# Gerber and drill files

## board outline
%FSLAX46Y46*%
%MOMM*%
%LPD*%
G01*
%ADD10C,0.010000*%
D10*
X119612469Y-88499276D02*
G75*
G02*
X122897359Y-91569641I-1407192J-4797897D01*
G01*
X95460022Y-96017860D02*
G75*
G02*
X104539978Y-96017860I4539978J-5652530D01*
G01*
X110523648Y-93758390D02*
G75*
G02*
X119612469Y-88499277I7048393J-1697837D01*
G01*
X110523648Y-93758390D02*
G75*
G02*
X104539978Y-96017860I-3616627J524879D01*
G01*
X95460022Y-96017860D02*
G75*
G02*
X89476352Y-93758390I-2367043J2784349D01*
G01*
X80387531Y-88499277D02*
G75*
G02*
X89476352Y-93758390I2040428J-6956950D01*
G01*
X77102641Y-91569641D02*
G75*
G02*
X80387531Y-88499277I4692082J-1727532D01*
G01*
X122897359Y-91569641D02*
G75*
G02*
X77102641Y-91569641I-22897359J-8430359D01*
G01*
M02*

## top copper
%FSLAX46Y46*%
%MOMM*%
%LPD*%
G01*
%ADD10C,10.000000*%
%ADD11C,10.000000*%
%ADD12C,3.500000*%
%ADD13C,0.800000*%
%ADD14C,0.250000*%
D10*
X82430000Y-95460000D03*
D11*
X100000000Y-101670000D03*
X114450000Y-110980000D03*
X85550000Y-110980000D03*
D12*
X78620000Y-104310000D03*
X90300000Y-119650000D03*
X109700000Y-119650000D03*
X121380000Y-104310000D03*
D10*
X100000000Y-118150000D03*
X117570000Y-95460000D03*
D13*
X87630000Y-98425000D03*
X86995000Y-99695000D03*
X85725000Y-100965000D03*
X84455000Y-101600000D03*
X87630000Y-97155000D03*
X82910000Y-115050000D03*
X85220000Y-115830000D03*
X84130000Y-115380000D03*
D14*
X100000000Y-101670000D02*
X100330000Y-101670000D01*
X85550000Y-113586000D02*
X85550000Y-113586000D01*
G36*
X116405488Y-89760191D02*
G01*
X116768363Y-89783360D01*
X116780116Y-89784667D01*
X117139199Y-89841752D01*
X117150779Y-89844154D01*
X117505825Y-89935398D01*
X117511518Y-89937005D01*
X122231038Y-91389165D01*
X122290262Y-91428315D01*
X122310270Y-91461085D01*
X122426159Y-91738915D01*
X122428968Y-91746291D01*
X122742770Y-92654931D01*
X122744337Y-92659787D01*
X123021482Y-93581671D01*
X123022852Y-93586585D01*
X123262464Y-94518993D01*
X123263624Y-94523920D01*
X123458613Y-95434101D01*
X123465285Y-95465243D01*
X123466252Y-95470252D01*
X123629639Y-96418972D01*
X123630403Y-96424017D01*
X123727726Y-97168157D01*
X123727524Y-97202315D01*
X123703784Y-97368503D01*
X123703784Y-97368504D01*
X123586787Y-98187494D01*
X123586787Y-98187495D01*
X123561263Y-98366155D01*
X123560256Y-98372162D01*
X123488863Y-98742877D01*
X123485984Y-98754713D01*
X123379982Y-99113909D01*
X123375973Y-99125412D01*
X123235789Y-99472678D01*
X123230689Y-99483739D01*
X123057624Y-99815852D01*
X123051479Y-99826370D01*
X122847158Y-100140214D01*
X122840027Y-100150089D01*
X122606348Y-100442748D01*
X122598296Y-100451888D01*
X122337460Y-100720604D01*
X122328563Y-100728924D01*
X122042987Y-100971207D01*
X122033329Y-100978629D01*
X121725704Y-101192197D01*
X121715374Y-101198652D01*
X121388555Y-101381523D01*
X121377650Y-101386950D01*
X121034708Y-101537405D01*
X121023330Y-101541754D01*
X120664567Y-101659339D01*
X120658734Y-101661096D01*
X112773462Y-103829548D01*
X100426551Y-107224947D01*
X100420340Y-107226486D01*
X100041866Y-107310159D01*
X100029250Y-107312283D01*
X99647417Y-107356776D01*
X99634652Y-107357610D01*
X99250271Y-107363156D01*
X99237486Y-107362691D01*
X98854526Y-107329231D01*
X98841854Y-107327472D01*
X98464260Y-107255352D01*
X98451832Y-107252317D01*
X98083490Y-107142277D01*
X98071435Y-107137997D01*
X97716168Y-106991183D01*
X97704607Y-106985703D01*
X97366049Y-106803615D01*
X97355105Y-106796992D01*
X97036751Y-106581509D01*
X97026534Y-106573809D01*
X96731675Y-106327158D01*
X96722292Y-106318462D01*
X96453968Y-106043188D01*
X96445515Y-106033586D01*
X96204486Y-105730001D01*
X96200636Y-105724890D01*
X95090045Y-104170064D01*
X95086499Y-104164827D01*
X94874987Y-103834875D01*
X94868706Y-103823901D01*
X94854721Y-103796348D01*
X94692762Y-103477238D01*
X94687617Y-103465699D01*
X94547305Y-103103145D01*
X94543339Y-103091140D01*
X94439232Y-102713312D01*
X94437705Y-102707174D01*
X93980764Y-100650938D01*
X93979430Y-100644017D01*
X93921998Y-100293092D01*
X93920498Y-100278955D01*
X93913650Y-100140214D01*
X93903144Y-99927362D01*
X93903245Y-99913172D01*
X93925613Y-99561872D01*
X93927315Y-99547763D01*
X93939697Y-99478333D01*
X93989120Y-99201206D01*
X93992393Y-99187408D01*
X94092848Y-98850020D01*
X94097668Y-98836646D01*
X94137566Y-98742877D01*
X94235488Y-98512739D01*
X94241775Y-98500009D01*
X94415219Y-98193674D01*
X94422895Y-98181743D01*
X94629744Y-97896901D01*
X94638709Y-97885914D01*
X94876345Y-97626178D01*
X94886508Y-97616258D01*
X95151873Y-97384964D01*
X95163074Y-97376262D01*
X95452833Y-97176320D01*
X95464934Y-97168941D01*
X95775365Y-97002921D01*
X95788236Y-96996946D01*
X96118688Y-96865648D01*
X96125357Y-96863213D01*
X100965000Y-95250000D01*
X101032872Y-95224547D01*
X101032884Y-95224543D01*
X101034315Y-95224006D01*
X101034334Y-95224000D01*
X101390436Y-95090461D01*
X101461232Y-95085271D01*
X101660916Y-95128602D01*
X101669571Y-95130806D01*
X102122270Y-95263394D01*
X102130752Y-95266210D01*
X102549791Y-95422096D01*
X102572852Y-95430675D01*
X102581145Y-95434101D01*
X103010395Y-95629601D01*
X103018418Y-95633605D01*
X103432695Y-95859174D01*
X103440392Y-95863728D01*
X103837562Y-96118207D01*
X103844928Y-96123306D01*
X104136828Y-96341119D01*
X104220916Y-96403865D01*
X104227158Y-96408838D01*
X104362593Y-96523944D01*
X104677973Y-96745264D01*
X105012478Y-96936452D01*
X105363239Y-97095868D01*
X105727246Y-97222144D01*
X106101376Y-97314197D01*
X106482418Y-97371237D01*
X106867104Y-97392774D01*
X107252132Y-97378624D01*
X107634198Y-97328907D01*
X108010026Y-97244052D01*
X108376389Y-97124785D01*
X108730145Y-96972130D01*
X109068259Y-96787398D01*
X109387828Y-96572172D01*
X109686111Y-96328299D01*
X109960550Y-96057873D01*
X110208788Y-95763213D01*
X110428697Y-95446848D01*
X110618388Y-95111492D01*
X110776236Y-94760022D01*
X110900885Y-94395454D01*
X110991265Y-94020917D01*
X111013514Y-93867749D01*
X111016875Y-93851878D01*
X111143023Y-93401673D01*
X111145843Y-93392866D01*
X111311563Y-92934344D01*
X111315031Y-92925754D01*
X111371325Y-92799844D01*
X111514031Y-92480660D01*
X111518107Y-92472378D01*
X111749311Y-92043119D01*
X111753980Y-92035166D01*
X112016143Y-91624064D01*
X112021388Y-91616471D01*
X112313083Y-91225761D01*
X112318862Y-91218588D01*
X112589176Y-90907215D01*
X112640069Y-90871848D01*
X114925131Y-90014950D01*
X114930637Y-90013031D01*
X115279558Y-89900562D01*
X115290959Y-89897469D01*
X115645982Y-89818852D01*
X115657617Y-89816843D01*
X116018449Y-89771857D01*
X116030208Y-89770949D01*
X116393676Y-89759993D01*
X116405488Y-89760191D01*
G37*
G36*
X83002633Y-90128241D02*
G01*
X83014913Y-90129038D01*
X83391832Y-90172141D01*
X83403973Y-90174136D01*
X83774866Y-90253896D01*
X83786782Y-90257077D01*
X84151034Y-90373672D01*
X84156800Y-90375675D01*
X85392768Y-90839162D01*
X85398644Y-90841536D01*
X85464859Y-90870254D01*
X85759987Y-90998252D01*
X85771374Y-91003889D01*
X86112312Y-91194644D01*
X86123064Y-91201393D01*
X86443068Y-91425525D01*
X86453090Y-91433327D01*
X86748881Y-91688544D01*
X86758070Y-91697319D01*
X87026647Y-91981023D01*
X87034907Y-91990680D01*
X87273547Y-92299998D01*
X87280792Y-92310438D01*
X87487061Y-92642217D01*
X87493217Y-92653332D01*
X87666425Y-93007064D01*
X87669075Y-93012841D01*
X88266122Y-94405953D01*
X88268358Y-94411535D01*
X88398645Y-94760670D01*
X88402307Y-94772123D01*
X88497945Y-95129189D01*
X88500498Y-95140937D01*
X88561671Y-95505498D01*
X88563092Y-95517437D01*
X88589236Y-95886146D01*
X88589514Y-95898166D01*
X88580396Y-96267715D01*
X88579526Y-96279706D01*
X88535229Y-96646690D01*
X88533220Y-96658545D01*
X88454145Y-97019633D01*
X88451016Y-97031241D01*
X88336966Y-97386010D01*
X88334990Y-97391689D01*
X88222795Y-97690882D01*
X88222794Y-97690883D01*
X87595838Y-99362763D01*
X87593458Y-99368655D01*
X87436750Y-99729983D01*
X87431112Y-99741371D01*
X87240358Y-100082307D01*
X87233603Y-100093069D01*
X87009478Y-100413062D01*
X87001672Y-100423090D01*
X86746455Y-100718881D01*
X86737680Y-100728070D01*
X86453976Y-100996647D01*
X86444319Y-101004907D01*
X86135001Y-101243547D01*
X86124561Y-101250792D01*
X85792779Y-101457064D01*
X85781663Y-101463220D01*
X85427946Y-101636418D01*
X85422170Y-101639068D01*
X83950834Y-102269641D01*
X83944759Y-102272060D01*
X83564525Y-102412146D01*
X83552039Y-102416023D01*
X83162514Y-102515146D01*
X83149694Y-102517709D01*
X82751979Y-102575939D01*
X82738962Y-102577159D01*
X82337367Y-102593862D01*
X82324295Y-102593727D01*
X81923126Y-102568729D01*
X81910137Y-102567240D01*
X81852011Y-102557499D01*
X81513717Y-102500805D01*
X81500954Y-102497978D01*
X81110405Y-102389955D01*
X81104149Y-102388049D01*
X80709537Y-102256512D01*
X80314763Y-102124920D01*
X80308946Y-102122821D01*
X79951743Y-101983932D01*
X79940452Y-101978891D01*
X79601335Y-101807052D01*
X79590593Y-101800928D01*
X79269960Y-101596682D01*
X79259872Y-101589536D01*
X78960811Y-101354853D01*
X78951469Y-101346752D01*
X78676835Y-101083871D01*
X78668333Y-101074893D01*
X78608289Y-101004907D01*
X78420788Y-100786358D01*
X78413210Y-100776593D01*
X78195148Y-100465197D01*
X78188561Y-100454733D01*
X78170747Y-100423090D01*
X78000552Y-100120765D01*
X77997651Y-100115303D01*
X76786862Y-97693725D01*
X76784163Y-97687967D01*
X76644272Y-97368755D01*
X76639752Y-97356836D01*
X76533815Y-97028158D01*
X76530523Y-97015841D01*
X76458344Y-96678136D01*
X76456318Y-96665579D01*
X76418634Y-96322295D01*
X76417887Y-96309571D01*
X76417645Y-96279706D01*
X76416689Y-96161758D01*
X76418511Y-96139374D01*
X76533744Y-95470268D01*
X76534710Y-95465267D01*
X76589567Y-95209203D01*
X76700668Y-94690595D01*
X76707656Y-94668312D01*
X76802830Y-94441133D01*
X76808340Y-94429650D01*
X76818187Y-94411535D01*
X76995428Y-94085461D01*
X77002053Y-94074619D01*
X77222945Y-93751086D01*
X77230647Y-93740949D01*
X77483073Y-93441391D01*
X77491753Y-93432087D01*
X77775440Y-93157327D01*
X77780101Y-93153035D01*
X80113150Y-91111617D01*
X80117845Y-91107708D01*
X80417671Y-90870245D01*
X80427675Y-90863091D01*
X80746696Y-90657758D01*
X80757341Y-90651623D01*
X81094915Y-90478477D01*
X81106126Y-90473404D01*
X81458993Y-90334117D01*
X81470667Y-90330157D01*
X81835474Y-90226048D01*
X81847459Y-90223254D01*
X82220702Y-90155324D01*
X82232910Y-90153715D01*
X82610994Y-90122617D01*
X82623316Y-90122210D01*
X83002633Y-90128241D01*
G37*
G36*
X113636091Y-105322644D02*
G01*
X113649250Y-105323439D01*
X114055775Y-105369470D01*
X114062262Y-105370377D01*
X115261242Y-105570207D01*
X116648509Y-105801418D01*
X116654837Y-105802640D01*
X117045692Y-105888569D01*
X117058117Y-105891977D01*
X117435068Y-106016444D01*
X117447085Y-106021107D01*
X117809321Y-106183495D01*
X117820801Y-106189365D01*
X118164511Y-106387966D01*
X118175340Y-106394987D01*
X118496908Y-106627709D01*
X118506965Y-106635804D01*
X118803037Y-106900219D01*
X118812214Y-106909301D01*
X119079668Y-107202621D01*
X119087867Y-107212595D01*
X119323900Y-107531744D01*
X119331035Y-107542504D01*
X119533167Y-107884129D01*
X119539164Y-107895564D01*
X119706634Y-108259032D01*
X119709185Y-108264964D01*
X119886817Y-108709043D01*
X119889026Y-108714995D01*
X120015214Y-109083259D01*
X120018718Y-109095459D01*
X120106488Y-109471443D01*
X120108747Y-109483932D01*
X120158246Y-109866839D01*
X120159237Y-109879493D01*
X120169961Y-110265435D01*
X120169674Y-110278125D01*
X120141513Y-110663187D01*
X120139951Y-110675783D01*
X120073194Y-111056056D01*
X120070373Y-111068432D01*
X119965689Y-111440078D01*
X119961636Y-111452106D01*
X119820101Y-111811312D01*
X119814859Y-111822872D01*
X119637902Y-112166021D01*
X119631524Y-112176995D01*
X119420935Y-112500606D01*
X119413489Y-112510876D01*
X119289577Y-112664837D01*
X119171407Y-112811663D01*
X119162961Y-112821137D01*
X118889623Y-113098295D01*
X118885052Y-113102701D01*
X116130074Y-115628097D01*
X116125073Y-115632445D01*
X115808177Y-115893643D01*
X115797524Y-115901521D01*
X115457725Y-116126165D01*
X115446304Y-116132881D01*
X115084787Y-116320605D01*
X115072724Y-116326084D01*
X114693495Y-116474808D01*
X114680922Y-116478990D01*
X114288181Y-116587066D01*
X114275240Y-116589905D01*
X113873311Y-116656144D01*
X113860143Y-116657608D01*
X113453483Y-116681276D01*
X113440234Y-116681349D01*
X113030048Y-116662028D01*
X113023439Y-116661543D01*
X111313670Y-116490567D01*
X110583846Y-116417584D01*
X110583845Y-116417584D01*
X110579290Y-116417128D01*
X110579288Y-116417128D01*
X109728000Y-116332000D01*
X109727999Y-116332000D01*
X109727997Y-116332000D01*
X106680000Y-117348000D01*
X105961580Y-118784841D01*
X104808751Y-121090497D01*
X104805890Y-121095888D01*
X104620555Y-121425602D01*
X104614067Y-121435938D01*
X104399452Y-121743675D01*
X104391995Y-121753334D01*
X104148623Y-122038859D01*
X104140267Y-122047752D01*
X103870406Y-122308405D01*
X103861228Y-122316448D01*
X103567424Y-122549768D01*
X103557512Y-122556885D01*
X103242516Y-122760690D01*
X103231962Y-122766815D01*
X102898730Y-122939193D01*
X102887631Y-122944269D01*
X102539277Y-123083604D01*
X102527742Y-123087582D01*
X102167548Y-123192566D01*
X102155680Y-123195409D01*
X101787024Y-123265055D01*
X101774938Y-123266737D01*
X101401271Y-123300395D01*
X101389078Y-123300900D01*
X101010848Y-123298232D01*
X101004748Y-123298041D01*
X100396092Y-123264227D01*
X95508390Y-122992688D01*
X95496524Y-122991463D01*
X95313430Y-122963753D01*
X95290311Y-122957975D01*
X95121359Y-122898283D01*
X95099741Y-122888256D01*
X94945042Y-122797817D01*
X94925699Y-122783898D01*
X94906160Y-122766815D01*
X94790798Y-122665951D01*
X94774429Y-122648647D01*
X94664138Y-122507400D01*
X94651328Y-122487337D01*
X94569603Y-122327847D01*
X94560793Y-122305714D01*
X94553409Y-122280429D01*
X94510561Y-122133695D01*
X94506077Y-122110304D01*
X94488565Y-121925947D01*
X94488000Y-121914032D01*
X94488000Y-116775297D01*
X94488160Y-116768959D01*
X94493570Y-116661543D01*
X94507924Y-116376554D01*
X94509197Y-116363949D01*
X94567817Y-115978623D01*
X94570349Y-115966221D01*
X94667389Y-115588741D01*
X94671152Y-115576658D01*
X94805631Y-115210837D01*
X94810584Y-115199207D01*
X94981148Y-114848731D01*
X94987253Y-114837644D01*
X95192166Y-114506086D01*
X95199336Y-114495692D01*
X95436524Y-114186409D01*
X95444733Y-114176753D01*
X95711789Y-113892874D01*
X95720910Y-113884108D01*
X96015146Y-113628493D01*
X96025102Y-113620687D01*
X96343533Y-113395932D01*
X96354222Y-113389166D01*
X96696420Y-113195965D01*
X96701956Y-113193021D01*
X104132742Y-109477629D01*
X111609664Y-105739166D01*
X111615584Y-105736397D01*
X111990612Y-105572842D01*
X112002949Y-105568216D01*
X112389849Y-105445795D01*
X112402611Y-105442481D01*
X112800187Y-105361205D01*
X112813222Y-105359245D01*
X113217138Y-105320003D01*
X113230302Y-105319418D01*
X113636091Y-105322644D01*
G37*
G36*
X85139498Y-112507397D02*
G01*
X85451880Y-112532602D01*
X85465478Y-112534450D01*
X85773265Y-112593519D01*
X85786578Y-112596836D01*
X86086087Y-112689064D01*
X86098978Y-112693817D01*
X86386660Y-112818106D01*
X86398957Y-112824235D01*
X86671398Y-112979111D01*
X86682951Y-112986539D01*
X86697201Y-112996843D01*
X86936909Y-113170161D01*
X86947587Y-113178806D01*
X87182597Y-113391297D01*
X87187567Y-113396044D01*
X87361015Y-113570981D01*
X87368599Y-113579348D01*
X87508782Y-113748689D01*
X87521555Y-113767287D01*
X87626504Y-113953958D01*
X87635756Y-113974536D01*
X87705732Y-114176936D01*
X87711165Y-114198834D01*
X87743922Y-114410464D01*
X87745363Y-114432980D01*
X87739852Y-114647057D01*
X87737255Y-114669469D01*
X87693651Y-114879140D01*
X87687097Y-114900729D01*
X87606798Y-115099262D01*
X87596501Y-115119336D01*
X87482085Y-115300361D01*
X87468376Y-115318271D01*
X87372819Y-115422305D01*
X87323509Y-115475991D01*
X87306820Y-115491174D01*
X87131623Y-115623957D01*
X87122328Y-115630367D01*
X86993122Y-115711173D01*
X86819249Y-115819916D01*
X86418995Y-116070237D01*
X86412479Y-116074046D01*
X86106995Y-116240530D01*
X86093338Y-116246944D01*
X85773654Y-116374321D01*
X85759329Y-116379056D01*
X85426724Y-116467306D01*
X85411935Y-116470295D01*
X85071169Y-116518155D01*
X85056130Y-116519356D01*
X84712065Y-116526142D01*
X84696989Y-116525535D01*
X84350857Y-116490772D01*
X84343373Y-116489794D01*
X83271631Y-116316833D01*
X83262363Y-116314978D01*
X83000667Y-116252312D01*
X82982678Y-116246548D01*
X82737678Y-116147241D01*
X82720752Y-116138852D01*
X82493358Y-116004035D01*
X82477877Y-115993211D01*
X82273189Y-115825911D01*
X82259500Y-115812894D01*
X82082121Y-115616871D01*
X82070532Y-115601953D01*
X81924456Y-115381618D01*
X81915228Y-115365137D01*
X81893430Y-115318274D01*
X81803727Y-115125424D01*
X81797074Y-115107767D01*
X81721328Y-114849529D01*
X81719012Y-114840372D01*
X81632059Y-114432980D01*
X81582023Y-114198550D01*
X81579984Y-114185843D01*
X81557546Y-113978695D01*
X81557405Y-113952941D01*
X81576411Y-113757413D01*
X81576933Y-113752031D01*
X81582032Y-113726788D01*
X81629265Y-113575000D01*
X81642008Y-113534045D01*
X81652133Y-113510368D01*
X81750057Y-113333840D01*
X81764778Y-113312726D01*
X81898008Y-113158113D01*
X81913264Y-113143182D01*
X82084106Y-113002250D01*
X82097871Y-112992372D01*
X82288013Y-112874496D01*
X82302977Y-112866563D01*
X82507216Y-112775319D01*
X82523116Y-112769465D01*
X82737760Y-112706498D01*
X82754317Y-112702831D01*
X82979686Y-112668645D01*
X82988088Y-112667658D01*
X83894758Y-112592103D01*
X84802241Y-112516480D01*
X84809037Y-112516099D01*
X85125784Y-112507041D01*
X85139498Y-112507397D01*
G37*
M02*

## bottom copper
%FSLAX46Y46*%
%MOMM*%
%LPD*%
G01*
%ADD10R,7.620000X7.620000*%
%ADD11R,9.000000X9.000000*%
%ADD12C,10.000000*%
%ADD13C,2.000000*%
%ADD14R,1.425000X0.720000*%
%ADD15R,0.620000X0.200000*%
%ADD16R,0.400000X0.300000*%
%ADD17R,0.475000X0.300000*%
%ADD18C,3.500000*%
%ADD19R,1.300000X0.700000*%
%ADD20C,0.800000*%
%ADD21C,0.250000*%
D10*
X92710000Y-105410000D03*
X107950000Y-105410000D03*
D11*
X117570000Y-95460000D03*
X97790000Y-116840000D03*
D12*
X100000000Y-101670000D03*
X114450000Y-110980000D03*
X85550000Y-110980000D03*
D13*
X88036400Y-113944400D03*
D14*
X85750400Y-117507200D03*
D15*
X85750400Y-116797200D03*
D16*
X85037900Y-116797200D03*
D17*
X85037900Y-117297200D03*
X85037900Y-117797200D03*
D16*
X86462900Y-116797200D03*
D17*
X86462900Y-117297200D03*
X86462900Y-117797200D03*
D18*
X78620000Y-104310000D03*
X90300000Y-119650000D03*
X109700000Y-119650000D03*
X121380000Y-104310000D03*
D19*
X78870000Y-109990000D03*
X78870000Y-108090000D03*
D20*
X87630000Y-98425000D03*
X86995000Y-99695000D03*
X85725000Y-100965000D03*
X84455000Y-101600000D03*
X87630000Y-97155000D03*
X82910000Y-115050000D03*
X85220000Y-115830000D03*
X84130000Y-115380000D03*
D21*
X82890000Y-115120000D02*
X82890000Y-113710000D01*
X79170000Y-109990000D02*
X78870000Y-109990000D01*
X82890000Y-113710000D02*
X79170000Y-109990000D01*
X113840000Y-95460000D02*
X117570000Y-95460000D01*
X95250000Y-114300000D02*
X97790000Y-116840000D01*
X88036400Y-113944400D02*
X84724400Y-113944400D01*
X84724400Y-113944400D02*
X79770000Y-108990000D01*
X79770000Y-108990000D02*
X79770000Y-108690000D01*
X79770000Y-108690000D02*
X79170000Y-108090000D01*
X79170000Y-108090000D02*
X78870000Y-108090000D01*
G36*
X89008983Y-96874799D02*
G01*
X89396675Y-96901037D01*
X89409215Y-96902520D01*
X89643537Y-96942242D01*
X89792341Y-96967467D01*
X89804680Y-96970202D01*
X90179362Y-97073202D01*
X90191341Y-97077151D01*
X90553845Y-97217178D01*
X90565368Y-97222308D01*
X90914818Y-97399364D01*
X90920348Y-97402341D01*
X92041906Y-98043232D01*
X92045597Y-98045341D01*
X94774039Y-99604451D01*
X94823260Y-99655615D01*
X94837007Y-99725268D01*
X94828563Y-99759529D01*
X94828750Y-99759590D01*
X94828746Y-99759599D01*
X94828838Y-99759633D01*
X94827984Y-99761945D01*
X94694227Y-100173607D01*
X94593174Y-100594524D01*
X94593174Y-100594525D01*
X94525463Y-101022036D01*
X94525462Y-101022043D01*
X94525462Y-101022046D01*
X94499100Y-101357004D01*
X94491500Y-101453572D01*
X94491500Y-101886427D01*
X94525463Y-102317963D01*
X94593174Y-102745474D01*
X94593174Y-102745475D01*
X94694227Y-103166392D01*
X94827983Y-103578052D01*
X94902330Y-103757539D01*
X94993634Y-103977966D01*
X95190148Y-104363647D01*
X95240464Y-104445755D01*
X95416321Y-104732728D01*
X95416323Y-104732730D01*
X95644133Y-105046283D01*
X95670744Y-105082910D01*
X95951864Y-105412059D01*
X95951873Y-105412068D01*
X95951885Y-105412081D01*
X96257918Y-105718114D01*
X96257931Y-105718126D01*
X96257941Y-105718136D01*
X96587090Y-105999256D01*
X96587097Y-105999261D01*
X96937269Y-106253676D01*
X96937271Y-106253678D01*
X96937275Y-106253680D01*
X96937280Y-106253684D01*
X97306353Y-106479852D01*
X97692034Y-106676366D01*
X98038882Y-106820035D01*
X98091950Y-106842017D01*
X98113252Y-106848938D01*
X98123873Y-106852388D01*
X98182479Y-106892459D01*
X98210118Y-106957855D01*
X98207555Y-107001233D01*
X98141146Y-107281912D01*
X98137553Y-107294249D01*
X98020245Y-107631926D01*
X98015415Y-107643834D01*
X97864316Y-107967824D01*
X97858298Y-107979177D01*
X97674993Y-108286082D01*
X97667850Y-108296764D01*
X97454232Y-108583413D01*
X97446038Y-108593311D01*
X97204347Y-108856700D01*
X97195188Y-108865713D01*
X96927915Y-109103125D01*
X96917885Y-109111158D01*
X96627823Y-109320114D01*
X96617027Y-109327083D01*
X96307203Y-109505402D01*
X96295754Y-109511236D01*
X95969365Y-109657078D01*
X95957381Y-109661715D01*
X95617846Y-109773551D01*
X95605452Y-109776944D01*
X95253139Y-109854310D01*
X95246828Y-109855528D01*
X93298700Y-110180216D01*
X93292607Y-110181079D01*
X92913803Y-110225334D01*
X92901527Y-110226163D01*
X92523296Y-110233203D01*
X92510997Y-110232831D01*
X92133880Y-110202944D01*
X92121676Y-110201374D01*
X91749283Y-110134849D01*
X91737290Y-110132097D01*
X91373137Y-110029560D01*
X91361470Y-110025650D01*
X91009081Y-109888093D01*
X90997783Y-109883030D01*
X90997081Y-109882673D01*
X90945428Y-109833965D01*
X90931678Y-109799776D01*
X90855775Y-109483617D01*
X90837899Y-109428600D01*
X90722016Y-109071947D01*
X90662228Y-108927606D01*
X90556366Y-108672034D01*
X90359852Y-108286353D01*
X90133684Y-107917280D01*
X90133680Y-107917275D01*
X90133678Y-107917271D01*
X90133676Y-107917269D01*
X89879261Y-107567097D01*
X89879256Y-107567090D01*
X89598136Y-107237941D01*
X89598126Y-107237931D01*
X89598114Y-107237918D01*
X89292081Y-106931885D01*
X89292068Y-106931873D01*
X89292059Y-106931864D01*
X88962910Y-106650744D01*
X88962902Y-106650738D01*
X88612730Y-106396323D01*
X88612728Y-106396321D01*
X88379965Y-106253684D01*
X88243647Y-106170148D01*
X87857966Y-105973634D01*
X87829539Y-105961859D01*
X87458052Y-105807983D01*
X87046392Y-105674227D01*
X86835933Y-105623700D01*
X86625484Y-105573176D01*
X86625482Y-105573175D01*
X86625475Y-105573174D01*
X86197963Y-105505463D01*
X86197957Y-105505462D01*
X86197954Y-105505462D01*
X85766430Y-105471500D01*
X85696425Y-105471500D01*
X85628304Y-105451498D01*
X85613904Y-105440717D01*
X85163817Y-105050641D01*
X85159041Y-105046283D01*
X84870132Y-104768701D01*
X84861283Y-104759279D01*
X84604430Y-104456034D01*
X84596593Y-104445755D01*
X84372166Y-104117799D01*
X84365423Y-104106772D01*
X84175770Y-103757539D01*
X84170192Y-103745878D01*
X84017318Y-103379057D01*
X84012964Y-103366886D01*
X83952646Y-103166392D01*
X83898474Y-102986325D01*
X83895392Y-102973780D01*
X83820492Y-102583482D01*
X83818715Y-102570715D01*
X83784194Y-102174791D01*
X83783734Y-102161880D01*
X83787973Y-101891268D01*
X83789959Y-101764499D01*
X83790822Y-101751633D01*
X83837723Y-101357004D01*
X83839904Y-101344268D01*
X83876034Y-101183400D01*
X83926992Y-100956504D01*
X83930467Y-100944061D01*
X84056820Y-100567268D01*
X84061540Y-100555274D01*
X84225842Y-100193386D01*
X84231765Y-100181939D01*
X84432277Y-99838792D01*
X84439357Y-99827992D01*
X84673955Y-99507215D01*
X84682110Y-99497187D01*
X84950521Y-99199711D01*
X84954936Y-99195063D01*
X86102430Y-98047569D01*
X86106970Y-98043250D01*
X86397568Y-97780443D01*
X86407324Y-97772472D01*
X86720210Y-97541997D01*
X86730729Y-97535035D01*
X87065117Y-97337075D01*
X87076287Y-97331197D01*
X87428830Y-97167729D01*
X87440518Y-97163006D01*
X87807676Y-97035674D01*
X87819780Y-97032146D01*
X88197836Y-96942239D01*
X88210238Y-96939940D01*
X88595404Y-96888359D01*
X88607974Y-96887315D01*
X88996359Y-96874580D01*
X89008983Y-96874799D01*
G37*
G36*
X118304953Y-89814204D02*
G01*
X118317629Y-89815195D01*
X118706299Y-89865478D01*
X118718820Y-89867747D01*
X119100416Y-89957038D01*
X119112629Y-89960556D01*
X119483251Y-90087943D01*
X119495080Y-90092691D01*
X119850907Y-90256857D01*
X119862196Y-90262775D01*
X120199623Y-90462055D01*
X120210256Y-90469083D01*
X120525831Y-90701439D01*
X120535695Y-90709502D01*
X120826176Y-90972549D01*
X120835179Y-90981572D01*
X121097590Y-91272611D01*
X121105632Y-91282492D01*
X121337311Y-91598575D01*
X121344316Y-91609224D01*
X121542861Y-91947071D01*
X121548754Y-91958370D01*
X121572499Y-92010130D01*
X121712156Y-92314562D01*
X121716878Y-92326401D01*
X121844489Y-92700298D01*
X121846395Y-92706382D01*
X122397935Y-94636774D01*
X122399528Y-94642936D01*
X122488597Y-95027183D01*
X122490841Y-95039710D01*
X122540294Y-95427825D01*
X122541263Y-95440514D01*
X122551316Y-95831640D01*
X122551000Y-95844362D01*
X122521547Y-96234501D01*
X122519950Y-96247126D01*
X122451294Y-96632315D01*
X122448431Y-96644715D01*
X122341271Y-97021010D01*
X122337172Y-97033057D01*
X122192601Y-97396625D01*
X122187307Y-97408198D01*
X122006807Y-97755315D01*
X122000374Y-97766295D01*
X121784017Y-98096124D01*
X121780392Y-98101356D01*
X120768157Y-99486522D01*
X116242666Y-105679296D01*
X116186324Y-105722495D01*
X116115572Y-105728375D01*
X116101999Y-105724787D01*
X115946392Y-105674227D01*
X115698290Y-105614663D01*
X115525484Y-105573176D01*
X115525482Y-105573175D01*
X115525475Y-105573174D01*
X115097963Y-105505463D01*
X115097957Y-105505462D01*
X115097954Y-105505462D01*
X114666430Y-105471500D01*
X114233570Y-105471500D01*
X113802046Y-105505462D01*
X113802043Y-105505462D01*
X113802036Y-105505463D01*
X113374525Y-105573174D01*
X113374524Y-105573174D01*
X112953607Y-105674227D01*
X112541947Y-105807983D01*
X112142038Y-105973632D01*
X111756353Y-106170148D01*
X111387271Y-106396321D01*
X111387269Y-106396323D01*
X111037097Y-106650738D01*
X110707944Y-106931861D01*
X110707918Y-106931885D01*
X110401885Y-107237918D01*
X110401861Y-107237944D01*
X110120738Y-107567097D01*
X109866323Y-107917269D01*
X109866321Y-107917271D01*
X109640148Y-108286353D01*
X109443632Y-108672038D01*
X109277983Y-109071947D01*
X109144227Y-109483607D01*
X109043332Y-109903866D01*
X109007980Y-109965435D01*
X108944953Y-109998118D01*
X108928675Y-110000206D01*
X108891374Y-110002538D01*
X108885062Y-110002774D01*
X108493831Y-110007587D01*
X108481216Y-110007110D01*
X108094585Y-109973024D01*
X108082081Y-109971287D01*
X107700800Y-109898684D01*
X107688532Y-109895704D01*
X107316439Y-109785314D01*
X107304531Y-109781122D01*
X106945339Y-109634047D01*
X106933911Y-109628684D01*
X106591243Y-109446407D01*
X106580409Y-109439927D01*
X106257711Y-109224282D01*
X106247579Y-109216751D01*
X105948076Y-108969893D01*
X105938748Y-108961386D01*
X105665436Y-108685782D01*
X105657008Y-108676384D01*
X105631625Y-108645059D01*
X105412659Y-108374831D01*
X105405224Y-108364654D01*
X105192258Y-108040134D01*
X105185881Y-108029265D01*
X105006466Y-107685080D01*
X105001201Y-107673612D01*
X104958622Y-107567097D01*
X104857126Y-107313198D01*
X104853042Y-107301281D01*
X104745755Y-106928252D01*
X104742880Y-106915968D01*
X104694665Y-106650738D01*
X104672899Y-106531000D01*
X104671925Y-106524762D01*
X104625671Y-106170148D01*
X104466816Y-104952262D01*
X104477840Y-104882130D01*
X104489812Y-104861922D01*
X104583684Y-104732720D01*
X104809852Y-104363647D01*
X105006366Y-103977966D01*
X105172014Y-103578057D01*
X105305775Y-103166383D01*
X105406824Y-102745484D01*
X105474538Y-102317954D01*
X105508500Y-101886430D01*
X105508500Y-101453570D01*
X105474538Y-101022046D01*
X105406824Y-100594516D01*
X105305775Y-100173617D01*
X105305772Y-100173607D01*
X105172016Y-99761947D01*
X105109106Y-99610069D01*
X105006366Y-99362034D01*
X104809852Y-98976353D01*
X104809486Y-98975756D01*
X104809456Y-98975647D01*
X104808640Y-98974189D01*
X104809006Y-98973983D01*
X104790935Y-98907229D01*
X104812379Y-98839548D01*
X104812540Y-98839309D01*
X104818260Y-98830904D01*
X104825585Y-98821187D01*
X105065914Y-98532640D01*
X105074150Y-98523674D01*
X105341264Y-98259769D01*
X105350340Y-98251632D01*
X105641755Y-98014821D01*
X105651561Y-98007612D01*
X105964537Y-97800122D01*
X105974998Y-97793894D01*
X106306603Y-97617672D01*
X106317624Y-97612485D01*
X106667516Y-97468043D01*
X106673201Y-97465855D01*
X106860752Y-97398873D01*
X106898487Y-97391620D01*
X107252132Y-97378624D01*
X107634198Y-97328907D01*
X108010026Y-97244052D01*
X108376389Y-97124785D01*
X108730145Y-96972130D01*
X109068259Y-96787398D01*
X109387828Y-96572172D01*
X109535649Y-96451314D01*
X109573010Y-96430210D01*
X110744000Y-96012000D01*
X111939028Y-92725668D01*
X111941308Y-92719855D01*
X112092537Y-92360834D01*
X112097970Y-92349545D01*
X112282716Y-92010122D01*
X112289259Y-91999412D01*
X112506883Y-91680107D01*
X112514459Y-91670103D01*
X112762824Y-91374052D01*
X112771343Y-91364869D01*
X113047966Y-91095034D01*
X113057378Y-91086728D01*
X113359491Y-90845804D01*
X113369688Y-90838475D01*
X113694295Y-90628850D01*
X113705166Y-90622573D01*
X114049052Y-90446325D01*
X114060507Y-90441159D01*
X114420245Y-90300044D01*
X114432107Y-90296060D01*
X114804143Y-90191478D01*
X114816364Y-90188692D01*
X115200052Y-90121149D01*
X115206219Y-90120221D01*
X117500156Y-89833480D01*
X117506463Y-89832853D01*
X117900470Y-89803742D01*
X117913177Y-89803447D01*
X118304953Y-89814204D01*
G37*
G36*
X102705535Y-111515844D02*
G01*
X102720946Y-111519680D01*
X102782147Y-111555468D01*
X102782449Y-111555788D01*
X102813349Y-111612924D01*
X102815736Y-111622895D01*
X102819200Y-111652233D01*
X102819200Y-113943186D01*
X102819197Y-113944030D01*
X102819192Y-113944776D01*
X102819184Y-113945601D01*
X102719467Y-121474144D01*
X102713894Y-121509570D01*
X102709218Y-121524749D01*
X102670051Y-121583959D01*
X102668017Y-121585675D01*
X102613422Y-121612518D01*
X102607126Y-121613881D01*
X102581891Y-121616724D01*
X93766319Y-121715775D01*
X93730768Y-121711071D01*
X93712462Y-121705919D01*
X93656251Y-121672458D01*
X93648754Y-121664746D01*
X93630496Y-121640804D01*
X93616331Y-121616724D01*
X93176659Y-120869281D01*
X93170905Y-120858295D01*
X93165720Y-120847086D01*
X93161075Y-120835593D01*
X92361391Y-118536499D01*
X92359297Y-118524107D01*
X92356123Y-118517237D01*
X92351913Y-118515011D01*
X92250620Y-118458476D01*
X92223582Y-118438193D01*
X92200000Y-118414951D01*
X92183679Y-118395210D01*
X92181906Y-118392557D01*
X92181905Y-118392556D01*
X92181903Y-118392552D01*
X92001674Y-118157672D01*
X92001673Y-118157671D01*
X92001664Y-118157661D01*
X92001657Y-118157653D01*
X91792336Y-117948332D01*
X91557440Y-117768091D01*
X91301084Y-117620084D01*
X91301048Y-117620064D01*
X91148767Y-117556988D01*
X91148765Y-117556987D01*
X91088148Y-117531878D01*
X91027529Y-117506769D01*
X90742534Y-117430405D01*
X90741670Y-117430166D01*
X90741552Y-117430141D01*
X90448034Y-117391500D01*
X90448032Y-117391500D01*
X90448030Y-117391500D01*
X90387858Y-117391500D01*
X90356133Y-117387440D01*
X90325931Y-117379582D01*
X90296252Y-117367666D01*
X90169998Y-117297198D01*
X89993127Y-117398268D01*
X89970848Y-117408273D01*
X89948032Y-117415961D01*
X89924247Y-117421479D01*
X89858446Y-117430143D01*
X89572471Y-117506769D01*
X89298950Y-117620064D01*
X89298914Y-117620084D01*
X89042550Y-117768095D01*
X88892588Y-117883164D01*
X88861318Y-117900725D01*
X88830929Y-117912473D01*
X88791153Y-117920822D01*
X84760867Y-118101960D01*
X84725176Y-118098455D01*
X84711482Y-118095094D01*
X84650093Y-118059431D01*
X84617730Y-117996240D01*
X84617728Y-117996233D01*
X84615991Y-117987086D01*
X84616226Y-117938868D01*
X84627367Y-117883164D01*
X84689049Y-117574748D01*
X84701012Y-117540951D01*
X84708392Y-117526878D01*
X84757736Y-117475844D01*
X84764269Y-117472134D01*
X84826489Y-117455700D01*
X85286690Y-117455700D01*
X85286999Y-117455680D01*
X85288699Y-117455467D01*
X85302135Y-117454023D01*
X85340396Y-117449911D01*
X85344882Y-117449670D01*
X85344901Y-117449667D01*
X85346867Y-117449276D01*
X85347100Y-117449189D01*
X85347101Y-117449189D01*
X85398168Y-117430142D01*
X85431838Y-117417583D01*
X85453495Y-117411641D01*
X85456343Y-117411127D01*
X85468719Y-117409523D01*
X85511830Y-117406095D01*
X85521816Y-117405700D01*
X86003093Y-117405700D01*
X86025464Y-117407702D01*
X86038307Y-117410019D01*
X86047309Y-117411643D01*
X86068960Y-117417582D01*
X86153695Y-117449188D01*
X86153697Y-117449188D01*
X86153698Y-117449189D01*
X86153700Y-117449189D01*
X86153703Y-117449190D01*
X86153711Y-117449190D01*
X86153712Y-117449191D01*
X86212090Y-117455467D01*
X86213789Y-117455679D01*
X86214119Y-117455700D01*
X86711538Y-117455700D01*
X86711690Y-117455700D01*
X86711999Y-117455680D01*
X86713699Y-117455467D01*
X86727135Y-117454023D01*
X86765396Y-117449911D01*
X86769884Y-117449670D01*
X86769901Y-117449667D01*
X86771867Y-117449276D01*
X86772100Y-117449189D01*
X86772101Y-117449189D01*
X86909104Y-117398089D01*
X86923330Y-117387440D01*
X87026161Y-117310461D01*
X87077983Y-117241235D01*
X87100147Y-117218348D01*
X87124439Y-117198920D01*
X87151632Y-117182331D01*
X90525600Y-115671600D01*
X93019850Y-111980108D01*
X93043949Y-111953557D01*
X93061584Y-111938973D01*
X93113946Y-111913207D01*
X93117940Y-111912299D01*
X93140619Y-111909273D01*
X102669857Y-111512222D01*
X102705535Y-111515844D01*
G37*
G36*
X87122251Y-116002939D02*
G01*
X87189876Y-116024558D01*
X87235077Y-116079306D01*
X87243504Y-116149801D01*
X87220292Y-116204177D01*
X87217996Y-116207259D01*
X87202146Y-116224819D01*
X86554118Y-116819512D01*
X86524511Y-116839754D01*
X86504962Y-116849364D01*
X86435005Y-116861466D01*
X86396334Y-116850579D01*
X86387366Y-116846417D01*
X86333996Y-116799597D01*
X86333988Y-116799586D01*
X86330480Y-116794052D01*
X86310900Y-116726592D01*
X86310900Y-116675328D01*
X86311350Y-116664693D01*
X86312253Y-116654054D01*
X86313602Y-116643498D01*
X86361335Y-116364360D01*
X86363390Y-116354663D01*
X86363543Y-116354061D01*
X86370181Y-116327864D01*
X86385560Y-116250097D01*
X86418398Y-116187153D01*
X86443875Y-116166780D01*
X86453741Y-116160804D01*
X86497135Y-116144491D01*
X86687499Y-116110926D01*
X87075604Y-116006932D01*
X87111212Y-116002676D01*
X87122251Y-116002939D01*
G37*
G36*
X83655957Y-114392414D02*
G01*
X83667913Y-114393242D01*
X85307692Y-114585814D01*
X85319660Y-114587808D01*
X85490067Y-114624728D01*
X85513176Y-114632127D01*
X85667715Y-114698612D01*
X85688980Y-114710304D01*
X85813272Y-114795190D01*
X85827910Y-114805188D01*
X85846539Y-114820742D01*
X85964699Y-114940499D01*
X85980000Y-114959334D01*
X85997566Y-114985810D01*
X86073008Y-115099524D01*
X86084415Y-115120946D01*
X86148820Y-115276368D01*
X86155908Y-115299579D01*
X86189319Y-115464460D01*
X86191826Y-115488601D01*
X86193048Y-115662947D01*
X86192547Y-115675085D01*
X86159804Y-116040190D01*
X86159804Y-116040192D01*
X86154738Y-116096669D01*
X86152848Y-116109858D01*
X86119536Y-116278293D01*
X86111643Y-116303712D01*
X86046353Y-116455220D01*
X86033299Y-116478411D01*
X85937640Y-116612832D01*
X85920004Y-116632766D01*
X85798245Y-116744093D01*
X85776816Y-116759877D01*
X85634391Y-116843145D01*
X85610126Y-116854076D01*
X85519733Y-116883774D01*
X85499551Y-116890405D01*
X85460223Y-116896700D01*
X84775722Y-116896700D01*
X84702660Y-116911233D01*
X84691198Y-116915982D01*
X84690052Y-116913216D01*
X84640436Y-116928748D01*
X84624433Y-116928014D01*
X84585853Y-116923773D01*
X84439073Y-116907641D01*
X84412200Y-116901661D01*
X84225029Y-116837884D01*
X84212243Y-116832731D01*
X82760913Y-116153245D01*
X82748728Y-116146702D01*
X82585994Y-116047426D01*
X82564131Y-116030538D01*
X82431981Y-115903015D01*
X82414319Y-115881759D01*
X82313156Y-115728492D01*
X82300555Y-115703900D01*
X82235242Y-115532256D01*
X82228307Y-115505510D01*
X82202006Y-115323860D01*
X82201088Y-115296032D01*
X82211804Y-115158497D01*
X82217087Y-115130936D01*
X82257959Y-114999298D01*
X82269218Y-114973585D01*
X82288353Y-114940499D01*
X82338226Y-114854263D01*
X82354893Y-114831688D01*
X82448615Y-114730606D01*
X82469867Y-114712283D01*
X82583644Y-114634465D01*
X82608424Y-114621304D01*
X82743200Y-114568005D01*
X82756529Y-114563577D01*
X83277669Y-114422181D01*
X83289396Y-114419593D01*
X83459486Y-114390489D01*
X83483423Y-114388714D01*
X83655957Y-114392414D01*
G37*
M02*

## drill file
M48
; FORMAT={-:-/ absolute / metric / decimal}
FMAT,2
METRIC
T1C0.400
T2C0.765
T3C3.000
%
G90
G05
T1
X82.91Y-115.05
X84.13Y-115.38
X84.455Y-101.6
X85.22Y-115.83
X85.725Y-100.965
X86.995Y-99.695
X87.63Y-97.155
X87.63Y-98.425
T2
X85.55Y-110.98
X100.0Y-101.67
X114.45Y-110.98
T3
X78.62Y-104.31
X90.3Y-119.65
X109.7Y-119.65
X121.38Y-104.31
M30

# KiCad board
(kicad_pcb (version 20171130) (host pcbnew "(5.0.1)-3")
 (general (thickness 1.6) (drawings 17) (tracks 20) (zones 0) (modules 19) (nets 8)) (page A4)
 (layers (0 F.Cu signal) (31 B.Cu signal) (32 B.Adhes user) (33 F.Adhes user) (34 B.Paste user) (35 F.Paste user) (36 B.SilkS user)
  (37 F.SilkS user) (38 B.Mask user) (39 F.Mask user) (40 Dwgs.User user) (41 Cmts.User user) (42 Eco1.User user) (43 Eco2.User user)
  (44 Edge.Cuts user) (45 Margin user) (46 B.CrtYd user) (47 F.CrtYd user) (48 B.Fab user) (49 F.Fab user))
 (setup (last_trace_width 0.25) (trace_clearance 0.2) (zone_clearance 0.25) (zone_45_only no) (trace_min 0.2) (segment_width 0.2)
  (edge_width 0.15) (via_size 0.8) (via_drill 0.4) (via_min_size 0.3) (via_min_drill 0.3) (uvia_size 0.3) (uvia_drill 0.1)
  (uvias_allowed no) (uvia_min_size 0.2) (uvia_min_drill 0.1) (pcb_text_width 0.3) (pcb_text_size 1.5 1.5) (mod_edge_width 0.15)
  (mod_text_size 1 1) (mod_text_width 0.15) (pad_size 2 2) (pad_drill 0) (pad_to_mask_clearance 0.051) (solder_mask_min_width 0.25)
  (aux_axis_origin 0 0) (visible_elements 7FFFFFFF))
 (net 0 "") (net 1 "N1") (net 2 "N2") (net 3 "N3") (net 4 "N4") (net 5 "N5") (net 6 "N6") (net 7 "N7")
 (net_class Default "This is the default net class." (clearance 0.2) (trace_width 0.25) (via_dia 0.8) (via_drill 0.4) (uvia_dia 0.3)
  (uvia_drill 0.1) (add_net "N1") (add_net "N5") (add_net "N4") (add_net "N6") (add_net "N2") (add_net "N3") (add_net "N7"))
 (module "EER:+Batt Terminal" (layer F.Cu) (at 82.43 95.46)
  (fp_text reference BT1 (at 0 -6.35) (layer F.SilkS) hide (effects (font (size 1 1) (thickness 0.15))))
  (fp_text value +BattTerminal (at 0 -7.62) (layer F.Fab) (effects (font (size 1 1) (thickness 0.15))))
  (pad 1 smd circle (at 0 0) (size 10 10) (layers F.Cu F.Paste F.Mask) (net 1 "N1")))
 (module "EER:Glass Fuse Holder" (layer F.Cu) (at 111.76 101.6 180)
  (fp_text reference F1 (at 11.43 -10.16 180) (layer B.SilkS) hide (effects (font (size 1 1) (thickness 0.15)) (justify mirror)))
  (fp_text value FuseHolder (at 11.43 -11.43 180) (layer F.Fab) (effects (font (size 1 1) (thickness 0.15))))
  (pad 2 smd rect (at 19.05 -3.81 180) (size 7.62 7.62) (layers B.Cu B.Mask) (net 1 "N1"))
  (pad 1 smd rect (at 3.81 -3.81 180) (size 7.62 7.62) (layers B.Cu B.Mask) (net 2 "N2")))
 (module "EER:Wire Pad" (layer F.Cu) (at 112.49 100.54)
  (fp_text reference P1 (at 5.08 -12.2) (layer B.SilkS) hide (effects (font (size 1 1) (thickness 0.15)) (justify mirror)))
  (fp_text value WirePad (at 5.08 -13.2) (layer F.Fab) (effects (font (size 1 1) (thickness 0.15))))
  (pad 1 smd rect (at 5.08 -5.08) (size 9 9) (layers B.Cu B.Mask) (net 2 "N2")))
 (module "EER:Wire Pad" (layer F.Cu) (at 92.71 121.92)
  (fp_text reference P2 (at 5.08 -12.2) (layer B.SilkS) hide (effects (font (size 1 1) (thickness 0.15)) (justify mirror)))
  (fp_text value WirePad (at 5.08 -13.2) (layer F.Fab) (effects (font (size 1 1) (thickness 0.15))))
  (pad 1 smd rect (at 5.08 -5.08) (size 9 9) (layers B.Cu B.Mask) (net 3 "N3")))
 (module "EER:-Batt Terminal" (layer F.Cu) (at 100 101.67)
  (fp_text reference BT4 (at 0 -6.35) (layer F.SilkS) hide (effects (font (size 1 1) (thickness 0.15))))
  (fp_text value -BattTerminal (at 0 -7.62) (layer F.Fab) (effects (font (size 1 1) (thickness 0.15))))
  (pad 1 thru_hole circle (at 0 0) (size 10 10) (drill 0.765) (layers F.Cu F.Mask) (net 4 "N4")))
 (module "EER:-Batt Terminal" (layer F.Cu) (at 114.45 110.98)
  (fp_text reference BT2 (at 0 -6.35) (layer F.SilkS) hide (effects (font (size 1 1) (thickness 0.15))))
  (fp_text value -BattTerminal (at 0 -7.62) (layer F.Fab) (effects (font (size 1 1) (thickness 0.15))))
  (pad 1 thru_hole circle (at 0 0) (size 10 10) (drill 0.765) (layers F.Cu F.Mask) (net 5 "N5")))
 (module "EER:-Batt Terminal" (layer F.Cu) (at 85.55 110.98)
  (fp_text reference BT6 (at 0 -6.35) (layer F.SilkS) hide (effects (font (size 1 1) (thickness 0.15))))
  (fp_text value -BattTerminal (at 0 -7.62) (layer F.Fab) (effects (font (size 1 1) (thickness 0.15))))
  (pad 1 thru_hole circle (at 0 0) (size 10 10) (drill 0.765) (layers F.Cu F.Mask) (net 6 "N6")))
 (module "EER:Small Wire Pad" (layer F.Cu) (at 85.4964 116.4844)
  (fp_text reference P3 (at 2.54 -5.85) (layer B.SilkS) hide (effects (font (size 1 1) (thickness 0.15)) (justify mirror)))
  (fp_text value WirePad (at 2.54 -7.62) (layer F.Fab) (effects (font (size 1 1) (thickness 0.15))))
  (pad 1 smd circle (at 2.54 -2.54) (size 2 2) (layers B.Cu B.Paste B.Mask) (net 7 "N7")))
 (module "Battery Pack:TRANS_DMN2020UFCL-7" (layer F.Cu) (at 85.7504 117.2972 180)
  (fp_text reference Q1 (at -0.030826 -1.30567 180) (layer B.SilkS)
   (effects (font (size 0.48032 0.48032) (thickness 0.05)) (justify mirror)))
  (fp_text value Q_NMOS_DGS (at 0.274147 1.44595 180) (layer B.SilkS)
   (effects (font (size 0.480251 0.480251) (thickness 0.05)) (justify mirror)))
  (pad 1 smd rect (at 0 -0.21 180) (size 1.425 0.72) (layers B.Cu B.Paste B.Mask) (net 3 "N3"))
  (pad 3 smd rect (at 0 0.5 180) (size 0.62 0.2) (layers B.Cu B.Paste B.Mask) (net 6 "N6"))
  (pad 3 smd rect (at 0.7125 0.5 180) (size 0.4 0.3) (layers B.Cu B.Paste B.Mask) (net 6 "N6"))
  (pad 1 smd rect (at 0.7125 0 180) (size 0.475 0.3) (layers B.Cu B.Paste B.Mask) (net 3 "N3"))
  (pad 1 smd rect (at 0.7125 -0.5 180) (size 0.475 0.3) (layers B.Cu B.Paste B.Mask) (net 3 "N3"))
  (pad 2 smd rect (at -0.7125 0.5 180) (size 0.4 0.3) (layers B.Cu B.Paste B.Mask) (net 7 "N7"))
  (pad 1 smd rect (at -0.7125 0 180) (size 0.475 0.3) (layers B.Cu B.Paste B.Mask) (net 3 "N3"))
  (pad 1 smd rect (at -0.7125 -0.5 180) (size 0.475 0.3) (layers B.Cu B.Paste B.Mask) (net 3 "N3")))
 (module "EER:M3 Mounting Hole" (layer F.Cu) (at 78.62 104.31)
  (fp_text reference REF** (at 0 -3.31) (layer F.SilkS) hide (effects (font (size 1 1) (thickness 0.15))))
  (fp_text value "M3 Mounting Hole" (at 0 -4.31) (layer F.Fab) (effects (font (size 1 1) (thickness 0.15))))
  (pad 1 thru_hole circle (at 0 0) (size 3.5 3.5) (drill 3) (layers *.Cu *.Mask)))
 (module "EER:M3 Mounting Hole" (layer F.Cu) (at 90.3 119.65)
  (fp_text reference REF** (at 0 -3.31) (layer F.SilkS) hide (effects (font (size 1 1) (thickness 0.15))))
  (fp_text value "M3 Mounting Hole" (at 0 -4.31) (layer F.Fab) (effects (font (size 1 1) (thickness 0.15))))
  (pad 1 thru_hole circle (at 0 0) (size 3.5 3.5) (drill 3) (layers *.Cu *.Mask)))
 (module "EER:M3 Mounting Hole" (layer F.Cu) (at 109.7 119.65)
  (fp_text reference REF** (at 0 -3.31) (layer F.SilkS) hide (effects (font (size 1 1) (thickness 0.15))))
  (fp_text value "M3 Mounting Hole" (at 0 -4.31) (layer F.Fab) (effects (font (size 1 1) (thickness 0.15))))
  (pad 1 thru_hole circle (at 0 0) (size 3.5 3.5) (drill 3) (layers *.Cu *.Mask)))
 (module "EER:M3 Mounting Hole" (layer F.Cu) (at 121.38 104.31)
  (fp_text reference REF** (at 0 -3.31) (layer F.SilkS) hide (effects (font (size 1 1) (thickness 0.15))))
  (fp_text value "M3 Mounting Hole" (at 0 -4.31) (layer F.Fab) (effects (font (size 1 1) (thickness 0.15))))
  (pad 1 thru_hole circle (at 0 0) (size 3.5 3.5) (drill 3) (layers *.Cu *.Mask)))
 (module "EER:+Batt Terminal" (layer F.Cu) (at 100 118.15)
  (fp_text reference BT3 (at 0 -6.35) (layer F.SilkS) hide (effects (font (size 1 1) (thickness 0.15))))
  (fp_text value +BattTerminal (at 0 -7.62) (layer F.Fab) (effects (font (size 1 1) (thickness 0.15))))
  (pad 1 smd circle (at 0 0) (size 10 10) (layers F.Cu F.Paste F.Mask) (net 5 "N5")))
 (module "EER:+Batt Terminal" (layer F.Cu) (at 117.57 95.46)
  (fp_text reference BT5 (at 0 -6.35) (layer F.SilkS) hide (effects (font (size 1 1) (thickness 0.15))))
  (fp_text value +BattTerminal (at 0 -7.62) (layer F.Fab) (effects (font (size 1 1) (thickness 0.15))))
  (pad 1 smd circle (at 0 0) (size 10 10) (layers F.Cu F.Paste F.Mask) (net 4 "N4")))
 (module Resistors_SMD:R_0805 (layer B.Cu) (at 78.87 109.04 270)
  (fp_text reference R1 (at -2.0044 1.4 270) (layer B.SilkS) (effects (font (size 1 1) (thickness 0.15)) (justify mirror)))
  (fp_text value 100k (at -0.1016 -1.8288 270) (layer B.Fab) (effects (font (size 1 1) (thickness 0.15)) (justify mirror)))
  (pad 2 smd rect (at 0.95 0 270) (size 0.7 1.3) (layers B.Cu B.Paste B.Mask) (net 6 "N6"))
  (pad 1 smd rect (at -0.95 0 270) (size 0.7 1.3) (layers B.Cu B.Paste B.Mask) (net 7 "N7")))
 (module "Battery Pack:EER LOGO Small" (layer B.Cu) (at 81.9912 91.2876 180)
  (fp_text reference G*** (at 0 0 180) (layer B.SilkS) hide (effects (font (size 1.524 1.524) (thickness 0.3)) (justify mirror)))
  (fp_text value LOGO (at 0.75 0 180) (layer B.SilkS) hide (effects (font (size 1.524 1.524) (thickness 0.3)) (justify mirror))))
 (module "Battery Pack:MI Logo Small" (layer B.Cu) (at 86.0552 94.4372 180)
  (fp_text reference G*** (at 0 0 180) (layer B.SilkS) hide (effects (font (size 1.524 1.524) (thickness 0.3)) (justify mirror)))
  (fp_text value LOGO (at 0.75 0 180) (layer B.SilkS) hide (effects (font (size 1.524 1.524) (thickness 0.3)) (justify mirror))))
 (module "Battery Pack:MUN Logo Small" (layer B.Cu) (at 79.6036 94.1324 180)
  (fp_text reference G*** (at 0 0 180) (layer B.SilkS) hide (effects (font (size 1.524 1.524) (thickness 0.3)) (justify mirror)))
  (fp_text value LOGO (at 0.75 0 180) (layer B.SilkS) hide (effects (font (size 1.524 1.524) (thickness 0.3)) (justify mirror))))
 (gr_arc (start 118.205277 93.297173) (end 122.897359 91.569641) (angle -53.44121718) (layer Edge.Cuts) (width 0.01))
 (gr_arc (start 100 101.67039) (end 104.539978 96.01786) (angle -77.54121026) (layer Edge.Cuts) (width 0.01))
 (gr_arc (start 117.572041 95.456227) (end 119.612469 88.499277) (angle -92.80251328) (layer Edge.Cuts) (width 0.01))
 (gr_arc (start 106.907021 93.233511) (end 104.539978 96.01786) (angle -122.1110283) (layer Edge.Cuts) (width 0.01))
 (gr_arc (start 93.092979 93.233511) (end 89.476352 93.75839) (angle -122.1110283) (layer Edge.Cuts) (width 0.01))
 (gr_arc (start 82.427959 95.456227) (end 89.476352 93.75839) (angle -92.80251328) (layer Edge.Cuts) (width 0.01))
 (gr_arc (start 81.794723 93.297173) (end 80.387531 88.499277) (angle -53.44121718) (layer Edge.Cuts) (width 0.01))
 (gr_arc (start 100 100) (end 77.102641 91.569641) (angle -220.4254378) (layer Edge.Cuts) (width 0.01))
 (via (at 87.63 98.425) (size 0.8) (drill 0.4) (layers F.Cu B.Cu) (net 1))
 (via (at 86.995 99.695) (size 0.8) (drill 0.4) (layers F.Cu B.Cu) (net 1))
 (via (at 85.725 100.965) (size 0.8) (drill 0.4) (layers F.Cu B.Cu) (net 1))
 (via (at 84.455 101.6) (size 0.8) (drill 0.4) (layers F.Cu B.Cu) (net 1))
 (via (at 87.63 97.155) (size 0.8) (drill 0.4) (layers F.Cu B.Cu) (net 1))
 (segment (start 100 101.67) (end 100.33 101.67) (width 0.25) (layer F.Cu) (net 4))
 (via (at 82.91 115.05) (size 0.8) (drill 0.4) (layers F.Cu B.Cu) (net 6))
 (via (at 85.22 115.83) (size 0.8) (drill 0.4) (layers F.Cu B.Cu) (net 6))
 (via (at 84.13 115.38) (size 0.8) (drill 0.4) (layers F.Cu B.Cu) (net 6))
 (segment (start 85.55 113.586) (end 85.55 113.586) (width 0.25) (layer F.Cu) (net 6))
 (segment (start 82.89 115.12) (end 82.89 113.71) (width 0.25) (layer B.Cu) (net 6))
 (segment (start 79.17 109.99) (end 78.87 109.99) (width 0.25) (layer B.Cu) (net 6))
 (segment (start 82.89 113.71) (end 79.17 109.99) (width 0.25) (layer B.Cu) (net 6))
 (segment (start 113.84 95.46) (end 117.57 95.46) (width 0.25) (layer B.Cu) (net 2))
 (segment (start 95.25 114.3) (end 97.79 116.84) (width 0.25) (layer B.Cu) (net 3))
 (segment (start 88.0364 113.9444) (end 84.7244 113.9444) (width 0.25) (layer B.Cu) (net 7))
 (segment (start 84.7244 113.9444) (end 79.77 108.99) (width 0.25) (layer B.Cu) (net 7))
 (segment (start 79.77 108.99) (end 79.77 108.69) (width 0.25) (layer B.Cu) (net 7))
 (segment (start 79.77 108.69) (end 79.17 108.09) (width 0.25) (layer B.Cu) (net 7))
 (segment (start 79.17 108.09) (end 78.87 108.09) (width 0.25) (layer B.Cu) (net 7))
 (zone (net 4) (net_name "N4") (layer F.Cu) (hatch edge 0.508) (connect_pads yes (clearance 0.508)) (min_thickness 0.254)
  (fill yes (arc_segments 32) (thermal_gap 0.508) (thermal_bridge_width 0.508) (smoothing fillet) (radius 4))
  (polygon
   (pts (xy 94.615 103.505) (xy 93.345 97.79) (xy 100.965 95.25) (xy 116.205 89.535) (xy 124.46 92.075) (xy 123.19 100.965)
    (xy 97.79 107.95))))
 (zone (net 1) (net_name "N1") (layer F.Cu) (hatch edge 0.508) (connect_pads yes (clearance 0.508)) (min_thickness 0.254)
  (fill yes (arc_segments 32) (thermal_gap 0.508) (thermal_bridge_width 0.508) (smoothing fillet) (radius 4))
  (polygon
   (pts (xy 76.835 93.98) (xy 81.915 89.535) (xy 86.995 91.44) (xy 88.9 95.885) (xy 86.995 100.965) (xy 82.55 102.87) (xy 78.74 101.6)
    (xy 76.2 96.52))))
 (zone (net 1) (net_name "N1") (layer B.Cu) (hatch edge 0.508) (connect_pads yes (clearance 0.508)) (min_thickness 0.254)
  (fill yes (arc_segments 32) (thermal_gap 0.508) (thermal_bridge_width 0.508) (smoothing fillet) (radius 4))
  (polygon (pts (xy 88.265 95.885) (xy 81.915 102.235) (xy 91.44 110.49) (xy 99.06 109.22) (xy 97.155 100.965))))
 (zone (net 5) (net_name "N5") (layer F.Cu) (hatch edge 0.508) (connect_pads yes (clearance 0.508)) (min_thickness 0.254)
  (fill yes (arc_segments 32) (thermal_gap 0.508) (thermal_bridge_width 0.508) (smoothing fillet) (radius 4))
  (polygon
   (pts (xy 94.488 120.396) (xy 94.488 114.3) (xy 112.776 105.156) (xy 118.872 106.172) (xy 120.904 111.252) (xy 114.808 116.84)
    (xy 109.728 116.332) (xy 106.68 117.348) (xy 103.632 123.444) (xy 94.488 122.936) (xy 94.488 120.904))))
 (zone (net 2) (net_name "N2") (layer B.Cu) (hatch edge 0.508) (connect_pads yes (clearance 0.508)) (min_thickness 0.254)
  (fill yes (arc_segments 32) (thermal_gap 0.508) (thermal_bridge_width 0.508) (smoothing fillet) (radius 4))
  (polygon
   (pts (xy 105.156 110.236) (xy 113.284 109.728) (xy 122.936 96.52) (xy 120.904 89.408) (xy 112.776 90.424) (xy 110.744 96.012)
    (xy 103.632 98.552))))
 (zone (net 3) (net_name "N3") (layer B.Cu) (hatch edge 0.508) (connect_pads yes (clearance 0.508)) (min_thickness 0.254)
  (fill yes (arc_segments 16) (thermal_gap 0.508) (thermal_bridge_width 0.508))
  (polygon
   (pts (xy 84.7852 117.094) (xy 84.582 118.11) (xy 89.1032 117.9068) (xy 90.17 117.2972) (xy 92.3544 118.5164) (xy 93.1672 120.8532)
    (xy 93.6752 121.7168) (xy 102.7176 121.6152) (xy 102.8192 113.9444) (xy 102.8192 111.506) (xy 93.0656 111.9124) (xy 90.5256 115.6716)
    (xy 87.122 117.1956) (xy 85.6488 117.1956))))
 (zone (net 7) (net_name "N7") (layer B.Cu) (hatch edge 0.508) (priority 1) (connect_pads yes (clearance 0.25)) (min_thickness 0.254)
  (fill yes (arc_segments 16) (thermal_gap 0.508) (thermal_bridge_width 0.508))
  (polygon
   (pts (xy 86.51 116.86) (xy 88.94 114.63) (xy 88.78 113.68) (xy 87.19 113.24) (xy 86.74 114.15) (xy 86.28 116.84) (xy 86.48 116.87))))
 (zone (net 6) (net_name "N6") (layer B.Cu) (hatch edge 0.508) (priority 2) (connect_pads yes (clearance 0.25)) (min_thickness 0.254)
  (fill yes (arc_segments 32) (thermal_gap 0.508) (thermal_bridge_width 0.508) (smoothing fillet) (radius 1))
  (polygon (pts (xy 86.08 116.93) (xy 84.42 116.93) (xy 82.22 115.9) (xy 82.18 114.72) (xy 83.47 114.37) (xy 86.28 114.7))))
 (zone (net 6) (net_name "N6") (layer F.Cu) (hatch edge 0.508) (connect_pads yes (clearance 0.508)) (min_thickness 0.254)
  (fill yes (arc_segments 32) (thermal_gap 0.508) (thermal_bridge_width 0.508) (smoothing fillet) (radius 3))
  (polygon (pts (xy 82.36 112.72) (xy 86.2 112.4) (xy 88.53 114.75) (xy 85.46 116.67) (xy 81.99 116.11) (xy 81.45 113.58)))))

